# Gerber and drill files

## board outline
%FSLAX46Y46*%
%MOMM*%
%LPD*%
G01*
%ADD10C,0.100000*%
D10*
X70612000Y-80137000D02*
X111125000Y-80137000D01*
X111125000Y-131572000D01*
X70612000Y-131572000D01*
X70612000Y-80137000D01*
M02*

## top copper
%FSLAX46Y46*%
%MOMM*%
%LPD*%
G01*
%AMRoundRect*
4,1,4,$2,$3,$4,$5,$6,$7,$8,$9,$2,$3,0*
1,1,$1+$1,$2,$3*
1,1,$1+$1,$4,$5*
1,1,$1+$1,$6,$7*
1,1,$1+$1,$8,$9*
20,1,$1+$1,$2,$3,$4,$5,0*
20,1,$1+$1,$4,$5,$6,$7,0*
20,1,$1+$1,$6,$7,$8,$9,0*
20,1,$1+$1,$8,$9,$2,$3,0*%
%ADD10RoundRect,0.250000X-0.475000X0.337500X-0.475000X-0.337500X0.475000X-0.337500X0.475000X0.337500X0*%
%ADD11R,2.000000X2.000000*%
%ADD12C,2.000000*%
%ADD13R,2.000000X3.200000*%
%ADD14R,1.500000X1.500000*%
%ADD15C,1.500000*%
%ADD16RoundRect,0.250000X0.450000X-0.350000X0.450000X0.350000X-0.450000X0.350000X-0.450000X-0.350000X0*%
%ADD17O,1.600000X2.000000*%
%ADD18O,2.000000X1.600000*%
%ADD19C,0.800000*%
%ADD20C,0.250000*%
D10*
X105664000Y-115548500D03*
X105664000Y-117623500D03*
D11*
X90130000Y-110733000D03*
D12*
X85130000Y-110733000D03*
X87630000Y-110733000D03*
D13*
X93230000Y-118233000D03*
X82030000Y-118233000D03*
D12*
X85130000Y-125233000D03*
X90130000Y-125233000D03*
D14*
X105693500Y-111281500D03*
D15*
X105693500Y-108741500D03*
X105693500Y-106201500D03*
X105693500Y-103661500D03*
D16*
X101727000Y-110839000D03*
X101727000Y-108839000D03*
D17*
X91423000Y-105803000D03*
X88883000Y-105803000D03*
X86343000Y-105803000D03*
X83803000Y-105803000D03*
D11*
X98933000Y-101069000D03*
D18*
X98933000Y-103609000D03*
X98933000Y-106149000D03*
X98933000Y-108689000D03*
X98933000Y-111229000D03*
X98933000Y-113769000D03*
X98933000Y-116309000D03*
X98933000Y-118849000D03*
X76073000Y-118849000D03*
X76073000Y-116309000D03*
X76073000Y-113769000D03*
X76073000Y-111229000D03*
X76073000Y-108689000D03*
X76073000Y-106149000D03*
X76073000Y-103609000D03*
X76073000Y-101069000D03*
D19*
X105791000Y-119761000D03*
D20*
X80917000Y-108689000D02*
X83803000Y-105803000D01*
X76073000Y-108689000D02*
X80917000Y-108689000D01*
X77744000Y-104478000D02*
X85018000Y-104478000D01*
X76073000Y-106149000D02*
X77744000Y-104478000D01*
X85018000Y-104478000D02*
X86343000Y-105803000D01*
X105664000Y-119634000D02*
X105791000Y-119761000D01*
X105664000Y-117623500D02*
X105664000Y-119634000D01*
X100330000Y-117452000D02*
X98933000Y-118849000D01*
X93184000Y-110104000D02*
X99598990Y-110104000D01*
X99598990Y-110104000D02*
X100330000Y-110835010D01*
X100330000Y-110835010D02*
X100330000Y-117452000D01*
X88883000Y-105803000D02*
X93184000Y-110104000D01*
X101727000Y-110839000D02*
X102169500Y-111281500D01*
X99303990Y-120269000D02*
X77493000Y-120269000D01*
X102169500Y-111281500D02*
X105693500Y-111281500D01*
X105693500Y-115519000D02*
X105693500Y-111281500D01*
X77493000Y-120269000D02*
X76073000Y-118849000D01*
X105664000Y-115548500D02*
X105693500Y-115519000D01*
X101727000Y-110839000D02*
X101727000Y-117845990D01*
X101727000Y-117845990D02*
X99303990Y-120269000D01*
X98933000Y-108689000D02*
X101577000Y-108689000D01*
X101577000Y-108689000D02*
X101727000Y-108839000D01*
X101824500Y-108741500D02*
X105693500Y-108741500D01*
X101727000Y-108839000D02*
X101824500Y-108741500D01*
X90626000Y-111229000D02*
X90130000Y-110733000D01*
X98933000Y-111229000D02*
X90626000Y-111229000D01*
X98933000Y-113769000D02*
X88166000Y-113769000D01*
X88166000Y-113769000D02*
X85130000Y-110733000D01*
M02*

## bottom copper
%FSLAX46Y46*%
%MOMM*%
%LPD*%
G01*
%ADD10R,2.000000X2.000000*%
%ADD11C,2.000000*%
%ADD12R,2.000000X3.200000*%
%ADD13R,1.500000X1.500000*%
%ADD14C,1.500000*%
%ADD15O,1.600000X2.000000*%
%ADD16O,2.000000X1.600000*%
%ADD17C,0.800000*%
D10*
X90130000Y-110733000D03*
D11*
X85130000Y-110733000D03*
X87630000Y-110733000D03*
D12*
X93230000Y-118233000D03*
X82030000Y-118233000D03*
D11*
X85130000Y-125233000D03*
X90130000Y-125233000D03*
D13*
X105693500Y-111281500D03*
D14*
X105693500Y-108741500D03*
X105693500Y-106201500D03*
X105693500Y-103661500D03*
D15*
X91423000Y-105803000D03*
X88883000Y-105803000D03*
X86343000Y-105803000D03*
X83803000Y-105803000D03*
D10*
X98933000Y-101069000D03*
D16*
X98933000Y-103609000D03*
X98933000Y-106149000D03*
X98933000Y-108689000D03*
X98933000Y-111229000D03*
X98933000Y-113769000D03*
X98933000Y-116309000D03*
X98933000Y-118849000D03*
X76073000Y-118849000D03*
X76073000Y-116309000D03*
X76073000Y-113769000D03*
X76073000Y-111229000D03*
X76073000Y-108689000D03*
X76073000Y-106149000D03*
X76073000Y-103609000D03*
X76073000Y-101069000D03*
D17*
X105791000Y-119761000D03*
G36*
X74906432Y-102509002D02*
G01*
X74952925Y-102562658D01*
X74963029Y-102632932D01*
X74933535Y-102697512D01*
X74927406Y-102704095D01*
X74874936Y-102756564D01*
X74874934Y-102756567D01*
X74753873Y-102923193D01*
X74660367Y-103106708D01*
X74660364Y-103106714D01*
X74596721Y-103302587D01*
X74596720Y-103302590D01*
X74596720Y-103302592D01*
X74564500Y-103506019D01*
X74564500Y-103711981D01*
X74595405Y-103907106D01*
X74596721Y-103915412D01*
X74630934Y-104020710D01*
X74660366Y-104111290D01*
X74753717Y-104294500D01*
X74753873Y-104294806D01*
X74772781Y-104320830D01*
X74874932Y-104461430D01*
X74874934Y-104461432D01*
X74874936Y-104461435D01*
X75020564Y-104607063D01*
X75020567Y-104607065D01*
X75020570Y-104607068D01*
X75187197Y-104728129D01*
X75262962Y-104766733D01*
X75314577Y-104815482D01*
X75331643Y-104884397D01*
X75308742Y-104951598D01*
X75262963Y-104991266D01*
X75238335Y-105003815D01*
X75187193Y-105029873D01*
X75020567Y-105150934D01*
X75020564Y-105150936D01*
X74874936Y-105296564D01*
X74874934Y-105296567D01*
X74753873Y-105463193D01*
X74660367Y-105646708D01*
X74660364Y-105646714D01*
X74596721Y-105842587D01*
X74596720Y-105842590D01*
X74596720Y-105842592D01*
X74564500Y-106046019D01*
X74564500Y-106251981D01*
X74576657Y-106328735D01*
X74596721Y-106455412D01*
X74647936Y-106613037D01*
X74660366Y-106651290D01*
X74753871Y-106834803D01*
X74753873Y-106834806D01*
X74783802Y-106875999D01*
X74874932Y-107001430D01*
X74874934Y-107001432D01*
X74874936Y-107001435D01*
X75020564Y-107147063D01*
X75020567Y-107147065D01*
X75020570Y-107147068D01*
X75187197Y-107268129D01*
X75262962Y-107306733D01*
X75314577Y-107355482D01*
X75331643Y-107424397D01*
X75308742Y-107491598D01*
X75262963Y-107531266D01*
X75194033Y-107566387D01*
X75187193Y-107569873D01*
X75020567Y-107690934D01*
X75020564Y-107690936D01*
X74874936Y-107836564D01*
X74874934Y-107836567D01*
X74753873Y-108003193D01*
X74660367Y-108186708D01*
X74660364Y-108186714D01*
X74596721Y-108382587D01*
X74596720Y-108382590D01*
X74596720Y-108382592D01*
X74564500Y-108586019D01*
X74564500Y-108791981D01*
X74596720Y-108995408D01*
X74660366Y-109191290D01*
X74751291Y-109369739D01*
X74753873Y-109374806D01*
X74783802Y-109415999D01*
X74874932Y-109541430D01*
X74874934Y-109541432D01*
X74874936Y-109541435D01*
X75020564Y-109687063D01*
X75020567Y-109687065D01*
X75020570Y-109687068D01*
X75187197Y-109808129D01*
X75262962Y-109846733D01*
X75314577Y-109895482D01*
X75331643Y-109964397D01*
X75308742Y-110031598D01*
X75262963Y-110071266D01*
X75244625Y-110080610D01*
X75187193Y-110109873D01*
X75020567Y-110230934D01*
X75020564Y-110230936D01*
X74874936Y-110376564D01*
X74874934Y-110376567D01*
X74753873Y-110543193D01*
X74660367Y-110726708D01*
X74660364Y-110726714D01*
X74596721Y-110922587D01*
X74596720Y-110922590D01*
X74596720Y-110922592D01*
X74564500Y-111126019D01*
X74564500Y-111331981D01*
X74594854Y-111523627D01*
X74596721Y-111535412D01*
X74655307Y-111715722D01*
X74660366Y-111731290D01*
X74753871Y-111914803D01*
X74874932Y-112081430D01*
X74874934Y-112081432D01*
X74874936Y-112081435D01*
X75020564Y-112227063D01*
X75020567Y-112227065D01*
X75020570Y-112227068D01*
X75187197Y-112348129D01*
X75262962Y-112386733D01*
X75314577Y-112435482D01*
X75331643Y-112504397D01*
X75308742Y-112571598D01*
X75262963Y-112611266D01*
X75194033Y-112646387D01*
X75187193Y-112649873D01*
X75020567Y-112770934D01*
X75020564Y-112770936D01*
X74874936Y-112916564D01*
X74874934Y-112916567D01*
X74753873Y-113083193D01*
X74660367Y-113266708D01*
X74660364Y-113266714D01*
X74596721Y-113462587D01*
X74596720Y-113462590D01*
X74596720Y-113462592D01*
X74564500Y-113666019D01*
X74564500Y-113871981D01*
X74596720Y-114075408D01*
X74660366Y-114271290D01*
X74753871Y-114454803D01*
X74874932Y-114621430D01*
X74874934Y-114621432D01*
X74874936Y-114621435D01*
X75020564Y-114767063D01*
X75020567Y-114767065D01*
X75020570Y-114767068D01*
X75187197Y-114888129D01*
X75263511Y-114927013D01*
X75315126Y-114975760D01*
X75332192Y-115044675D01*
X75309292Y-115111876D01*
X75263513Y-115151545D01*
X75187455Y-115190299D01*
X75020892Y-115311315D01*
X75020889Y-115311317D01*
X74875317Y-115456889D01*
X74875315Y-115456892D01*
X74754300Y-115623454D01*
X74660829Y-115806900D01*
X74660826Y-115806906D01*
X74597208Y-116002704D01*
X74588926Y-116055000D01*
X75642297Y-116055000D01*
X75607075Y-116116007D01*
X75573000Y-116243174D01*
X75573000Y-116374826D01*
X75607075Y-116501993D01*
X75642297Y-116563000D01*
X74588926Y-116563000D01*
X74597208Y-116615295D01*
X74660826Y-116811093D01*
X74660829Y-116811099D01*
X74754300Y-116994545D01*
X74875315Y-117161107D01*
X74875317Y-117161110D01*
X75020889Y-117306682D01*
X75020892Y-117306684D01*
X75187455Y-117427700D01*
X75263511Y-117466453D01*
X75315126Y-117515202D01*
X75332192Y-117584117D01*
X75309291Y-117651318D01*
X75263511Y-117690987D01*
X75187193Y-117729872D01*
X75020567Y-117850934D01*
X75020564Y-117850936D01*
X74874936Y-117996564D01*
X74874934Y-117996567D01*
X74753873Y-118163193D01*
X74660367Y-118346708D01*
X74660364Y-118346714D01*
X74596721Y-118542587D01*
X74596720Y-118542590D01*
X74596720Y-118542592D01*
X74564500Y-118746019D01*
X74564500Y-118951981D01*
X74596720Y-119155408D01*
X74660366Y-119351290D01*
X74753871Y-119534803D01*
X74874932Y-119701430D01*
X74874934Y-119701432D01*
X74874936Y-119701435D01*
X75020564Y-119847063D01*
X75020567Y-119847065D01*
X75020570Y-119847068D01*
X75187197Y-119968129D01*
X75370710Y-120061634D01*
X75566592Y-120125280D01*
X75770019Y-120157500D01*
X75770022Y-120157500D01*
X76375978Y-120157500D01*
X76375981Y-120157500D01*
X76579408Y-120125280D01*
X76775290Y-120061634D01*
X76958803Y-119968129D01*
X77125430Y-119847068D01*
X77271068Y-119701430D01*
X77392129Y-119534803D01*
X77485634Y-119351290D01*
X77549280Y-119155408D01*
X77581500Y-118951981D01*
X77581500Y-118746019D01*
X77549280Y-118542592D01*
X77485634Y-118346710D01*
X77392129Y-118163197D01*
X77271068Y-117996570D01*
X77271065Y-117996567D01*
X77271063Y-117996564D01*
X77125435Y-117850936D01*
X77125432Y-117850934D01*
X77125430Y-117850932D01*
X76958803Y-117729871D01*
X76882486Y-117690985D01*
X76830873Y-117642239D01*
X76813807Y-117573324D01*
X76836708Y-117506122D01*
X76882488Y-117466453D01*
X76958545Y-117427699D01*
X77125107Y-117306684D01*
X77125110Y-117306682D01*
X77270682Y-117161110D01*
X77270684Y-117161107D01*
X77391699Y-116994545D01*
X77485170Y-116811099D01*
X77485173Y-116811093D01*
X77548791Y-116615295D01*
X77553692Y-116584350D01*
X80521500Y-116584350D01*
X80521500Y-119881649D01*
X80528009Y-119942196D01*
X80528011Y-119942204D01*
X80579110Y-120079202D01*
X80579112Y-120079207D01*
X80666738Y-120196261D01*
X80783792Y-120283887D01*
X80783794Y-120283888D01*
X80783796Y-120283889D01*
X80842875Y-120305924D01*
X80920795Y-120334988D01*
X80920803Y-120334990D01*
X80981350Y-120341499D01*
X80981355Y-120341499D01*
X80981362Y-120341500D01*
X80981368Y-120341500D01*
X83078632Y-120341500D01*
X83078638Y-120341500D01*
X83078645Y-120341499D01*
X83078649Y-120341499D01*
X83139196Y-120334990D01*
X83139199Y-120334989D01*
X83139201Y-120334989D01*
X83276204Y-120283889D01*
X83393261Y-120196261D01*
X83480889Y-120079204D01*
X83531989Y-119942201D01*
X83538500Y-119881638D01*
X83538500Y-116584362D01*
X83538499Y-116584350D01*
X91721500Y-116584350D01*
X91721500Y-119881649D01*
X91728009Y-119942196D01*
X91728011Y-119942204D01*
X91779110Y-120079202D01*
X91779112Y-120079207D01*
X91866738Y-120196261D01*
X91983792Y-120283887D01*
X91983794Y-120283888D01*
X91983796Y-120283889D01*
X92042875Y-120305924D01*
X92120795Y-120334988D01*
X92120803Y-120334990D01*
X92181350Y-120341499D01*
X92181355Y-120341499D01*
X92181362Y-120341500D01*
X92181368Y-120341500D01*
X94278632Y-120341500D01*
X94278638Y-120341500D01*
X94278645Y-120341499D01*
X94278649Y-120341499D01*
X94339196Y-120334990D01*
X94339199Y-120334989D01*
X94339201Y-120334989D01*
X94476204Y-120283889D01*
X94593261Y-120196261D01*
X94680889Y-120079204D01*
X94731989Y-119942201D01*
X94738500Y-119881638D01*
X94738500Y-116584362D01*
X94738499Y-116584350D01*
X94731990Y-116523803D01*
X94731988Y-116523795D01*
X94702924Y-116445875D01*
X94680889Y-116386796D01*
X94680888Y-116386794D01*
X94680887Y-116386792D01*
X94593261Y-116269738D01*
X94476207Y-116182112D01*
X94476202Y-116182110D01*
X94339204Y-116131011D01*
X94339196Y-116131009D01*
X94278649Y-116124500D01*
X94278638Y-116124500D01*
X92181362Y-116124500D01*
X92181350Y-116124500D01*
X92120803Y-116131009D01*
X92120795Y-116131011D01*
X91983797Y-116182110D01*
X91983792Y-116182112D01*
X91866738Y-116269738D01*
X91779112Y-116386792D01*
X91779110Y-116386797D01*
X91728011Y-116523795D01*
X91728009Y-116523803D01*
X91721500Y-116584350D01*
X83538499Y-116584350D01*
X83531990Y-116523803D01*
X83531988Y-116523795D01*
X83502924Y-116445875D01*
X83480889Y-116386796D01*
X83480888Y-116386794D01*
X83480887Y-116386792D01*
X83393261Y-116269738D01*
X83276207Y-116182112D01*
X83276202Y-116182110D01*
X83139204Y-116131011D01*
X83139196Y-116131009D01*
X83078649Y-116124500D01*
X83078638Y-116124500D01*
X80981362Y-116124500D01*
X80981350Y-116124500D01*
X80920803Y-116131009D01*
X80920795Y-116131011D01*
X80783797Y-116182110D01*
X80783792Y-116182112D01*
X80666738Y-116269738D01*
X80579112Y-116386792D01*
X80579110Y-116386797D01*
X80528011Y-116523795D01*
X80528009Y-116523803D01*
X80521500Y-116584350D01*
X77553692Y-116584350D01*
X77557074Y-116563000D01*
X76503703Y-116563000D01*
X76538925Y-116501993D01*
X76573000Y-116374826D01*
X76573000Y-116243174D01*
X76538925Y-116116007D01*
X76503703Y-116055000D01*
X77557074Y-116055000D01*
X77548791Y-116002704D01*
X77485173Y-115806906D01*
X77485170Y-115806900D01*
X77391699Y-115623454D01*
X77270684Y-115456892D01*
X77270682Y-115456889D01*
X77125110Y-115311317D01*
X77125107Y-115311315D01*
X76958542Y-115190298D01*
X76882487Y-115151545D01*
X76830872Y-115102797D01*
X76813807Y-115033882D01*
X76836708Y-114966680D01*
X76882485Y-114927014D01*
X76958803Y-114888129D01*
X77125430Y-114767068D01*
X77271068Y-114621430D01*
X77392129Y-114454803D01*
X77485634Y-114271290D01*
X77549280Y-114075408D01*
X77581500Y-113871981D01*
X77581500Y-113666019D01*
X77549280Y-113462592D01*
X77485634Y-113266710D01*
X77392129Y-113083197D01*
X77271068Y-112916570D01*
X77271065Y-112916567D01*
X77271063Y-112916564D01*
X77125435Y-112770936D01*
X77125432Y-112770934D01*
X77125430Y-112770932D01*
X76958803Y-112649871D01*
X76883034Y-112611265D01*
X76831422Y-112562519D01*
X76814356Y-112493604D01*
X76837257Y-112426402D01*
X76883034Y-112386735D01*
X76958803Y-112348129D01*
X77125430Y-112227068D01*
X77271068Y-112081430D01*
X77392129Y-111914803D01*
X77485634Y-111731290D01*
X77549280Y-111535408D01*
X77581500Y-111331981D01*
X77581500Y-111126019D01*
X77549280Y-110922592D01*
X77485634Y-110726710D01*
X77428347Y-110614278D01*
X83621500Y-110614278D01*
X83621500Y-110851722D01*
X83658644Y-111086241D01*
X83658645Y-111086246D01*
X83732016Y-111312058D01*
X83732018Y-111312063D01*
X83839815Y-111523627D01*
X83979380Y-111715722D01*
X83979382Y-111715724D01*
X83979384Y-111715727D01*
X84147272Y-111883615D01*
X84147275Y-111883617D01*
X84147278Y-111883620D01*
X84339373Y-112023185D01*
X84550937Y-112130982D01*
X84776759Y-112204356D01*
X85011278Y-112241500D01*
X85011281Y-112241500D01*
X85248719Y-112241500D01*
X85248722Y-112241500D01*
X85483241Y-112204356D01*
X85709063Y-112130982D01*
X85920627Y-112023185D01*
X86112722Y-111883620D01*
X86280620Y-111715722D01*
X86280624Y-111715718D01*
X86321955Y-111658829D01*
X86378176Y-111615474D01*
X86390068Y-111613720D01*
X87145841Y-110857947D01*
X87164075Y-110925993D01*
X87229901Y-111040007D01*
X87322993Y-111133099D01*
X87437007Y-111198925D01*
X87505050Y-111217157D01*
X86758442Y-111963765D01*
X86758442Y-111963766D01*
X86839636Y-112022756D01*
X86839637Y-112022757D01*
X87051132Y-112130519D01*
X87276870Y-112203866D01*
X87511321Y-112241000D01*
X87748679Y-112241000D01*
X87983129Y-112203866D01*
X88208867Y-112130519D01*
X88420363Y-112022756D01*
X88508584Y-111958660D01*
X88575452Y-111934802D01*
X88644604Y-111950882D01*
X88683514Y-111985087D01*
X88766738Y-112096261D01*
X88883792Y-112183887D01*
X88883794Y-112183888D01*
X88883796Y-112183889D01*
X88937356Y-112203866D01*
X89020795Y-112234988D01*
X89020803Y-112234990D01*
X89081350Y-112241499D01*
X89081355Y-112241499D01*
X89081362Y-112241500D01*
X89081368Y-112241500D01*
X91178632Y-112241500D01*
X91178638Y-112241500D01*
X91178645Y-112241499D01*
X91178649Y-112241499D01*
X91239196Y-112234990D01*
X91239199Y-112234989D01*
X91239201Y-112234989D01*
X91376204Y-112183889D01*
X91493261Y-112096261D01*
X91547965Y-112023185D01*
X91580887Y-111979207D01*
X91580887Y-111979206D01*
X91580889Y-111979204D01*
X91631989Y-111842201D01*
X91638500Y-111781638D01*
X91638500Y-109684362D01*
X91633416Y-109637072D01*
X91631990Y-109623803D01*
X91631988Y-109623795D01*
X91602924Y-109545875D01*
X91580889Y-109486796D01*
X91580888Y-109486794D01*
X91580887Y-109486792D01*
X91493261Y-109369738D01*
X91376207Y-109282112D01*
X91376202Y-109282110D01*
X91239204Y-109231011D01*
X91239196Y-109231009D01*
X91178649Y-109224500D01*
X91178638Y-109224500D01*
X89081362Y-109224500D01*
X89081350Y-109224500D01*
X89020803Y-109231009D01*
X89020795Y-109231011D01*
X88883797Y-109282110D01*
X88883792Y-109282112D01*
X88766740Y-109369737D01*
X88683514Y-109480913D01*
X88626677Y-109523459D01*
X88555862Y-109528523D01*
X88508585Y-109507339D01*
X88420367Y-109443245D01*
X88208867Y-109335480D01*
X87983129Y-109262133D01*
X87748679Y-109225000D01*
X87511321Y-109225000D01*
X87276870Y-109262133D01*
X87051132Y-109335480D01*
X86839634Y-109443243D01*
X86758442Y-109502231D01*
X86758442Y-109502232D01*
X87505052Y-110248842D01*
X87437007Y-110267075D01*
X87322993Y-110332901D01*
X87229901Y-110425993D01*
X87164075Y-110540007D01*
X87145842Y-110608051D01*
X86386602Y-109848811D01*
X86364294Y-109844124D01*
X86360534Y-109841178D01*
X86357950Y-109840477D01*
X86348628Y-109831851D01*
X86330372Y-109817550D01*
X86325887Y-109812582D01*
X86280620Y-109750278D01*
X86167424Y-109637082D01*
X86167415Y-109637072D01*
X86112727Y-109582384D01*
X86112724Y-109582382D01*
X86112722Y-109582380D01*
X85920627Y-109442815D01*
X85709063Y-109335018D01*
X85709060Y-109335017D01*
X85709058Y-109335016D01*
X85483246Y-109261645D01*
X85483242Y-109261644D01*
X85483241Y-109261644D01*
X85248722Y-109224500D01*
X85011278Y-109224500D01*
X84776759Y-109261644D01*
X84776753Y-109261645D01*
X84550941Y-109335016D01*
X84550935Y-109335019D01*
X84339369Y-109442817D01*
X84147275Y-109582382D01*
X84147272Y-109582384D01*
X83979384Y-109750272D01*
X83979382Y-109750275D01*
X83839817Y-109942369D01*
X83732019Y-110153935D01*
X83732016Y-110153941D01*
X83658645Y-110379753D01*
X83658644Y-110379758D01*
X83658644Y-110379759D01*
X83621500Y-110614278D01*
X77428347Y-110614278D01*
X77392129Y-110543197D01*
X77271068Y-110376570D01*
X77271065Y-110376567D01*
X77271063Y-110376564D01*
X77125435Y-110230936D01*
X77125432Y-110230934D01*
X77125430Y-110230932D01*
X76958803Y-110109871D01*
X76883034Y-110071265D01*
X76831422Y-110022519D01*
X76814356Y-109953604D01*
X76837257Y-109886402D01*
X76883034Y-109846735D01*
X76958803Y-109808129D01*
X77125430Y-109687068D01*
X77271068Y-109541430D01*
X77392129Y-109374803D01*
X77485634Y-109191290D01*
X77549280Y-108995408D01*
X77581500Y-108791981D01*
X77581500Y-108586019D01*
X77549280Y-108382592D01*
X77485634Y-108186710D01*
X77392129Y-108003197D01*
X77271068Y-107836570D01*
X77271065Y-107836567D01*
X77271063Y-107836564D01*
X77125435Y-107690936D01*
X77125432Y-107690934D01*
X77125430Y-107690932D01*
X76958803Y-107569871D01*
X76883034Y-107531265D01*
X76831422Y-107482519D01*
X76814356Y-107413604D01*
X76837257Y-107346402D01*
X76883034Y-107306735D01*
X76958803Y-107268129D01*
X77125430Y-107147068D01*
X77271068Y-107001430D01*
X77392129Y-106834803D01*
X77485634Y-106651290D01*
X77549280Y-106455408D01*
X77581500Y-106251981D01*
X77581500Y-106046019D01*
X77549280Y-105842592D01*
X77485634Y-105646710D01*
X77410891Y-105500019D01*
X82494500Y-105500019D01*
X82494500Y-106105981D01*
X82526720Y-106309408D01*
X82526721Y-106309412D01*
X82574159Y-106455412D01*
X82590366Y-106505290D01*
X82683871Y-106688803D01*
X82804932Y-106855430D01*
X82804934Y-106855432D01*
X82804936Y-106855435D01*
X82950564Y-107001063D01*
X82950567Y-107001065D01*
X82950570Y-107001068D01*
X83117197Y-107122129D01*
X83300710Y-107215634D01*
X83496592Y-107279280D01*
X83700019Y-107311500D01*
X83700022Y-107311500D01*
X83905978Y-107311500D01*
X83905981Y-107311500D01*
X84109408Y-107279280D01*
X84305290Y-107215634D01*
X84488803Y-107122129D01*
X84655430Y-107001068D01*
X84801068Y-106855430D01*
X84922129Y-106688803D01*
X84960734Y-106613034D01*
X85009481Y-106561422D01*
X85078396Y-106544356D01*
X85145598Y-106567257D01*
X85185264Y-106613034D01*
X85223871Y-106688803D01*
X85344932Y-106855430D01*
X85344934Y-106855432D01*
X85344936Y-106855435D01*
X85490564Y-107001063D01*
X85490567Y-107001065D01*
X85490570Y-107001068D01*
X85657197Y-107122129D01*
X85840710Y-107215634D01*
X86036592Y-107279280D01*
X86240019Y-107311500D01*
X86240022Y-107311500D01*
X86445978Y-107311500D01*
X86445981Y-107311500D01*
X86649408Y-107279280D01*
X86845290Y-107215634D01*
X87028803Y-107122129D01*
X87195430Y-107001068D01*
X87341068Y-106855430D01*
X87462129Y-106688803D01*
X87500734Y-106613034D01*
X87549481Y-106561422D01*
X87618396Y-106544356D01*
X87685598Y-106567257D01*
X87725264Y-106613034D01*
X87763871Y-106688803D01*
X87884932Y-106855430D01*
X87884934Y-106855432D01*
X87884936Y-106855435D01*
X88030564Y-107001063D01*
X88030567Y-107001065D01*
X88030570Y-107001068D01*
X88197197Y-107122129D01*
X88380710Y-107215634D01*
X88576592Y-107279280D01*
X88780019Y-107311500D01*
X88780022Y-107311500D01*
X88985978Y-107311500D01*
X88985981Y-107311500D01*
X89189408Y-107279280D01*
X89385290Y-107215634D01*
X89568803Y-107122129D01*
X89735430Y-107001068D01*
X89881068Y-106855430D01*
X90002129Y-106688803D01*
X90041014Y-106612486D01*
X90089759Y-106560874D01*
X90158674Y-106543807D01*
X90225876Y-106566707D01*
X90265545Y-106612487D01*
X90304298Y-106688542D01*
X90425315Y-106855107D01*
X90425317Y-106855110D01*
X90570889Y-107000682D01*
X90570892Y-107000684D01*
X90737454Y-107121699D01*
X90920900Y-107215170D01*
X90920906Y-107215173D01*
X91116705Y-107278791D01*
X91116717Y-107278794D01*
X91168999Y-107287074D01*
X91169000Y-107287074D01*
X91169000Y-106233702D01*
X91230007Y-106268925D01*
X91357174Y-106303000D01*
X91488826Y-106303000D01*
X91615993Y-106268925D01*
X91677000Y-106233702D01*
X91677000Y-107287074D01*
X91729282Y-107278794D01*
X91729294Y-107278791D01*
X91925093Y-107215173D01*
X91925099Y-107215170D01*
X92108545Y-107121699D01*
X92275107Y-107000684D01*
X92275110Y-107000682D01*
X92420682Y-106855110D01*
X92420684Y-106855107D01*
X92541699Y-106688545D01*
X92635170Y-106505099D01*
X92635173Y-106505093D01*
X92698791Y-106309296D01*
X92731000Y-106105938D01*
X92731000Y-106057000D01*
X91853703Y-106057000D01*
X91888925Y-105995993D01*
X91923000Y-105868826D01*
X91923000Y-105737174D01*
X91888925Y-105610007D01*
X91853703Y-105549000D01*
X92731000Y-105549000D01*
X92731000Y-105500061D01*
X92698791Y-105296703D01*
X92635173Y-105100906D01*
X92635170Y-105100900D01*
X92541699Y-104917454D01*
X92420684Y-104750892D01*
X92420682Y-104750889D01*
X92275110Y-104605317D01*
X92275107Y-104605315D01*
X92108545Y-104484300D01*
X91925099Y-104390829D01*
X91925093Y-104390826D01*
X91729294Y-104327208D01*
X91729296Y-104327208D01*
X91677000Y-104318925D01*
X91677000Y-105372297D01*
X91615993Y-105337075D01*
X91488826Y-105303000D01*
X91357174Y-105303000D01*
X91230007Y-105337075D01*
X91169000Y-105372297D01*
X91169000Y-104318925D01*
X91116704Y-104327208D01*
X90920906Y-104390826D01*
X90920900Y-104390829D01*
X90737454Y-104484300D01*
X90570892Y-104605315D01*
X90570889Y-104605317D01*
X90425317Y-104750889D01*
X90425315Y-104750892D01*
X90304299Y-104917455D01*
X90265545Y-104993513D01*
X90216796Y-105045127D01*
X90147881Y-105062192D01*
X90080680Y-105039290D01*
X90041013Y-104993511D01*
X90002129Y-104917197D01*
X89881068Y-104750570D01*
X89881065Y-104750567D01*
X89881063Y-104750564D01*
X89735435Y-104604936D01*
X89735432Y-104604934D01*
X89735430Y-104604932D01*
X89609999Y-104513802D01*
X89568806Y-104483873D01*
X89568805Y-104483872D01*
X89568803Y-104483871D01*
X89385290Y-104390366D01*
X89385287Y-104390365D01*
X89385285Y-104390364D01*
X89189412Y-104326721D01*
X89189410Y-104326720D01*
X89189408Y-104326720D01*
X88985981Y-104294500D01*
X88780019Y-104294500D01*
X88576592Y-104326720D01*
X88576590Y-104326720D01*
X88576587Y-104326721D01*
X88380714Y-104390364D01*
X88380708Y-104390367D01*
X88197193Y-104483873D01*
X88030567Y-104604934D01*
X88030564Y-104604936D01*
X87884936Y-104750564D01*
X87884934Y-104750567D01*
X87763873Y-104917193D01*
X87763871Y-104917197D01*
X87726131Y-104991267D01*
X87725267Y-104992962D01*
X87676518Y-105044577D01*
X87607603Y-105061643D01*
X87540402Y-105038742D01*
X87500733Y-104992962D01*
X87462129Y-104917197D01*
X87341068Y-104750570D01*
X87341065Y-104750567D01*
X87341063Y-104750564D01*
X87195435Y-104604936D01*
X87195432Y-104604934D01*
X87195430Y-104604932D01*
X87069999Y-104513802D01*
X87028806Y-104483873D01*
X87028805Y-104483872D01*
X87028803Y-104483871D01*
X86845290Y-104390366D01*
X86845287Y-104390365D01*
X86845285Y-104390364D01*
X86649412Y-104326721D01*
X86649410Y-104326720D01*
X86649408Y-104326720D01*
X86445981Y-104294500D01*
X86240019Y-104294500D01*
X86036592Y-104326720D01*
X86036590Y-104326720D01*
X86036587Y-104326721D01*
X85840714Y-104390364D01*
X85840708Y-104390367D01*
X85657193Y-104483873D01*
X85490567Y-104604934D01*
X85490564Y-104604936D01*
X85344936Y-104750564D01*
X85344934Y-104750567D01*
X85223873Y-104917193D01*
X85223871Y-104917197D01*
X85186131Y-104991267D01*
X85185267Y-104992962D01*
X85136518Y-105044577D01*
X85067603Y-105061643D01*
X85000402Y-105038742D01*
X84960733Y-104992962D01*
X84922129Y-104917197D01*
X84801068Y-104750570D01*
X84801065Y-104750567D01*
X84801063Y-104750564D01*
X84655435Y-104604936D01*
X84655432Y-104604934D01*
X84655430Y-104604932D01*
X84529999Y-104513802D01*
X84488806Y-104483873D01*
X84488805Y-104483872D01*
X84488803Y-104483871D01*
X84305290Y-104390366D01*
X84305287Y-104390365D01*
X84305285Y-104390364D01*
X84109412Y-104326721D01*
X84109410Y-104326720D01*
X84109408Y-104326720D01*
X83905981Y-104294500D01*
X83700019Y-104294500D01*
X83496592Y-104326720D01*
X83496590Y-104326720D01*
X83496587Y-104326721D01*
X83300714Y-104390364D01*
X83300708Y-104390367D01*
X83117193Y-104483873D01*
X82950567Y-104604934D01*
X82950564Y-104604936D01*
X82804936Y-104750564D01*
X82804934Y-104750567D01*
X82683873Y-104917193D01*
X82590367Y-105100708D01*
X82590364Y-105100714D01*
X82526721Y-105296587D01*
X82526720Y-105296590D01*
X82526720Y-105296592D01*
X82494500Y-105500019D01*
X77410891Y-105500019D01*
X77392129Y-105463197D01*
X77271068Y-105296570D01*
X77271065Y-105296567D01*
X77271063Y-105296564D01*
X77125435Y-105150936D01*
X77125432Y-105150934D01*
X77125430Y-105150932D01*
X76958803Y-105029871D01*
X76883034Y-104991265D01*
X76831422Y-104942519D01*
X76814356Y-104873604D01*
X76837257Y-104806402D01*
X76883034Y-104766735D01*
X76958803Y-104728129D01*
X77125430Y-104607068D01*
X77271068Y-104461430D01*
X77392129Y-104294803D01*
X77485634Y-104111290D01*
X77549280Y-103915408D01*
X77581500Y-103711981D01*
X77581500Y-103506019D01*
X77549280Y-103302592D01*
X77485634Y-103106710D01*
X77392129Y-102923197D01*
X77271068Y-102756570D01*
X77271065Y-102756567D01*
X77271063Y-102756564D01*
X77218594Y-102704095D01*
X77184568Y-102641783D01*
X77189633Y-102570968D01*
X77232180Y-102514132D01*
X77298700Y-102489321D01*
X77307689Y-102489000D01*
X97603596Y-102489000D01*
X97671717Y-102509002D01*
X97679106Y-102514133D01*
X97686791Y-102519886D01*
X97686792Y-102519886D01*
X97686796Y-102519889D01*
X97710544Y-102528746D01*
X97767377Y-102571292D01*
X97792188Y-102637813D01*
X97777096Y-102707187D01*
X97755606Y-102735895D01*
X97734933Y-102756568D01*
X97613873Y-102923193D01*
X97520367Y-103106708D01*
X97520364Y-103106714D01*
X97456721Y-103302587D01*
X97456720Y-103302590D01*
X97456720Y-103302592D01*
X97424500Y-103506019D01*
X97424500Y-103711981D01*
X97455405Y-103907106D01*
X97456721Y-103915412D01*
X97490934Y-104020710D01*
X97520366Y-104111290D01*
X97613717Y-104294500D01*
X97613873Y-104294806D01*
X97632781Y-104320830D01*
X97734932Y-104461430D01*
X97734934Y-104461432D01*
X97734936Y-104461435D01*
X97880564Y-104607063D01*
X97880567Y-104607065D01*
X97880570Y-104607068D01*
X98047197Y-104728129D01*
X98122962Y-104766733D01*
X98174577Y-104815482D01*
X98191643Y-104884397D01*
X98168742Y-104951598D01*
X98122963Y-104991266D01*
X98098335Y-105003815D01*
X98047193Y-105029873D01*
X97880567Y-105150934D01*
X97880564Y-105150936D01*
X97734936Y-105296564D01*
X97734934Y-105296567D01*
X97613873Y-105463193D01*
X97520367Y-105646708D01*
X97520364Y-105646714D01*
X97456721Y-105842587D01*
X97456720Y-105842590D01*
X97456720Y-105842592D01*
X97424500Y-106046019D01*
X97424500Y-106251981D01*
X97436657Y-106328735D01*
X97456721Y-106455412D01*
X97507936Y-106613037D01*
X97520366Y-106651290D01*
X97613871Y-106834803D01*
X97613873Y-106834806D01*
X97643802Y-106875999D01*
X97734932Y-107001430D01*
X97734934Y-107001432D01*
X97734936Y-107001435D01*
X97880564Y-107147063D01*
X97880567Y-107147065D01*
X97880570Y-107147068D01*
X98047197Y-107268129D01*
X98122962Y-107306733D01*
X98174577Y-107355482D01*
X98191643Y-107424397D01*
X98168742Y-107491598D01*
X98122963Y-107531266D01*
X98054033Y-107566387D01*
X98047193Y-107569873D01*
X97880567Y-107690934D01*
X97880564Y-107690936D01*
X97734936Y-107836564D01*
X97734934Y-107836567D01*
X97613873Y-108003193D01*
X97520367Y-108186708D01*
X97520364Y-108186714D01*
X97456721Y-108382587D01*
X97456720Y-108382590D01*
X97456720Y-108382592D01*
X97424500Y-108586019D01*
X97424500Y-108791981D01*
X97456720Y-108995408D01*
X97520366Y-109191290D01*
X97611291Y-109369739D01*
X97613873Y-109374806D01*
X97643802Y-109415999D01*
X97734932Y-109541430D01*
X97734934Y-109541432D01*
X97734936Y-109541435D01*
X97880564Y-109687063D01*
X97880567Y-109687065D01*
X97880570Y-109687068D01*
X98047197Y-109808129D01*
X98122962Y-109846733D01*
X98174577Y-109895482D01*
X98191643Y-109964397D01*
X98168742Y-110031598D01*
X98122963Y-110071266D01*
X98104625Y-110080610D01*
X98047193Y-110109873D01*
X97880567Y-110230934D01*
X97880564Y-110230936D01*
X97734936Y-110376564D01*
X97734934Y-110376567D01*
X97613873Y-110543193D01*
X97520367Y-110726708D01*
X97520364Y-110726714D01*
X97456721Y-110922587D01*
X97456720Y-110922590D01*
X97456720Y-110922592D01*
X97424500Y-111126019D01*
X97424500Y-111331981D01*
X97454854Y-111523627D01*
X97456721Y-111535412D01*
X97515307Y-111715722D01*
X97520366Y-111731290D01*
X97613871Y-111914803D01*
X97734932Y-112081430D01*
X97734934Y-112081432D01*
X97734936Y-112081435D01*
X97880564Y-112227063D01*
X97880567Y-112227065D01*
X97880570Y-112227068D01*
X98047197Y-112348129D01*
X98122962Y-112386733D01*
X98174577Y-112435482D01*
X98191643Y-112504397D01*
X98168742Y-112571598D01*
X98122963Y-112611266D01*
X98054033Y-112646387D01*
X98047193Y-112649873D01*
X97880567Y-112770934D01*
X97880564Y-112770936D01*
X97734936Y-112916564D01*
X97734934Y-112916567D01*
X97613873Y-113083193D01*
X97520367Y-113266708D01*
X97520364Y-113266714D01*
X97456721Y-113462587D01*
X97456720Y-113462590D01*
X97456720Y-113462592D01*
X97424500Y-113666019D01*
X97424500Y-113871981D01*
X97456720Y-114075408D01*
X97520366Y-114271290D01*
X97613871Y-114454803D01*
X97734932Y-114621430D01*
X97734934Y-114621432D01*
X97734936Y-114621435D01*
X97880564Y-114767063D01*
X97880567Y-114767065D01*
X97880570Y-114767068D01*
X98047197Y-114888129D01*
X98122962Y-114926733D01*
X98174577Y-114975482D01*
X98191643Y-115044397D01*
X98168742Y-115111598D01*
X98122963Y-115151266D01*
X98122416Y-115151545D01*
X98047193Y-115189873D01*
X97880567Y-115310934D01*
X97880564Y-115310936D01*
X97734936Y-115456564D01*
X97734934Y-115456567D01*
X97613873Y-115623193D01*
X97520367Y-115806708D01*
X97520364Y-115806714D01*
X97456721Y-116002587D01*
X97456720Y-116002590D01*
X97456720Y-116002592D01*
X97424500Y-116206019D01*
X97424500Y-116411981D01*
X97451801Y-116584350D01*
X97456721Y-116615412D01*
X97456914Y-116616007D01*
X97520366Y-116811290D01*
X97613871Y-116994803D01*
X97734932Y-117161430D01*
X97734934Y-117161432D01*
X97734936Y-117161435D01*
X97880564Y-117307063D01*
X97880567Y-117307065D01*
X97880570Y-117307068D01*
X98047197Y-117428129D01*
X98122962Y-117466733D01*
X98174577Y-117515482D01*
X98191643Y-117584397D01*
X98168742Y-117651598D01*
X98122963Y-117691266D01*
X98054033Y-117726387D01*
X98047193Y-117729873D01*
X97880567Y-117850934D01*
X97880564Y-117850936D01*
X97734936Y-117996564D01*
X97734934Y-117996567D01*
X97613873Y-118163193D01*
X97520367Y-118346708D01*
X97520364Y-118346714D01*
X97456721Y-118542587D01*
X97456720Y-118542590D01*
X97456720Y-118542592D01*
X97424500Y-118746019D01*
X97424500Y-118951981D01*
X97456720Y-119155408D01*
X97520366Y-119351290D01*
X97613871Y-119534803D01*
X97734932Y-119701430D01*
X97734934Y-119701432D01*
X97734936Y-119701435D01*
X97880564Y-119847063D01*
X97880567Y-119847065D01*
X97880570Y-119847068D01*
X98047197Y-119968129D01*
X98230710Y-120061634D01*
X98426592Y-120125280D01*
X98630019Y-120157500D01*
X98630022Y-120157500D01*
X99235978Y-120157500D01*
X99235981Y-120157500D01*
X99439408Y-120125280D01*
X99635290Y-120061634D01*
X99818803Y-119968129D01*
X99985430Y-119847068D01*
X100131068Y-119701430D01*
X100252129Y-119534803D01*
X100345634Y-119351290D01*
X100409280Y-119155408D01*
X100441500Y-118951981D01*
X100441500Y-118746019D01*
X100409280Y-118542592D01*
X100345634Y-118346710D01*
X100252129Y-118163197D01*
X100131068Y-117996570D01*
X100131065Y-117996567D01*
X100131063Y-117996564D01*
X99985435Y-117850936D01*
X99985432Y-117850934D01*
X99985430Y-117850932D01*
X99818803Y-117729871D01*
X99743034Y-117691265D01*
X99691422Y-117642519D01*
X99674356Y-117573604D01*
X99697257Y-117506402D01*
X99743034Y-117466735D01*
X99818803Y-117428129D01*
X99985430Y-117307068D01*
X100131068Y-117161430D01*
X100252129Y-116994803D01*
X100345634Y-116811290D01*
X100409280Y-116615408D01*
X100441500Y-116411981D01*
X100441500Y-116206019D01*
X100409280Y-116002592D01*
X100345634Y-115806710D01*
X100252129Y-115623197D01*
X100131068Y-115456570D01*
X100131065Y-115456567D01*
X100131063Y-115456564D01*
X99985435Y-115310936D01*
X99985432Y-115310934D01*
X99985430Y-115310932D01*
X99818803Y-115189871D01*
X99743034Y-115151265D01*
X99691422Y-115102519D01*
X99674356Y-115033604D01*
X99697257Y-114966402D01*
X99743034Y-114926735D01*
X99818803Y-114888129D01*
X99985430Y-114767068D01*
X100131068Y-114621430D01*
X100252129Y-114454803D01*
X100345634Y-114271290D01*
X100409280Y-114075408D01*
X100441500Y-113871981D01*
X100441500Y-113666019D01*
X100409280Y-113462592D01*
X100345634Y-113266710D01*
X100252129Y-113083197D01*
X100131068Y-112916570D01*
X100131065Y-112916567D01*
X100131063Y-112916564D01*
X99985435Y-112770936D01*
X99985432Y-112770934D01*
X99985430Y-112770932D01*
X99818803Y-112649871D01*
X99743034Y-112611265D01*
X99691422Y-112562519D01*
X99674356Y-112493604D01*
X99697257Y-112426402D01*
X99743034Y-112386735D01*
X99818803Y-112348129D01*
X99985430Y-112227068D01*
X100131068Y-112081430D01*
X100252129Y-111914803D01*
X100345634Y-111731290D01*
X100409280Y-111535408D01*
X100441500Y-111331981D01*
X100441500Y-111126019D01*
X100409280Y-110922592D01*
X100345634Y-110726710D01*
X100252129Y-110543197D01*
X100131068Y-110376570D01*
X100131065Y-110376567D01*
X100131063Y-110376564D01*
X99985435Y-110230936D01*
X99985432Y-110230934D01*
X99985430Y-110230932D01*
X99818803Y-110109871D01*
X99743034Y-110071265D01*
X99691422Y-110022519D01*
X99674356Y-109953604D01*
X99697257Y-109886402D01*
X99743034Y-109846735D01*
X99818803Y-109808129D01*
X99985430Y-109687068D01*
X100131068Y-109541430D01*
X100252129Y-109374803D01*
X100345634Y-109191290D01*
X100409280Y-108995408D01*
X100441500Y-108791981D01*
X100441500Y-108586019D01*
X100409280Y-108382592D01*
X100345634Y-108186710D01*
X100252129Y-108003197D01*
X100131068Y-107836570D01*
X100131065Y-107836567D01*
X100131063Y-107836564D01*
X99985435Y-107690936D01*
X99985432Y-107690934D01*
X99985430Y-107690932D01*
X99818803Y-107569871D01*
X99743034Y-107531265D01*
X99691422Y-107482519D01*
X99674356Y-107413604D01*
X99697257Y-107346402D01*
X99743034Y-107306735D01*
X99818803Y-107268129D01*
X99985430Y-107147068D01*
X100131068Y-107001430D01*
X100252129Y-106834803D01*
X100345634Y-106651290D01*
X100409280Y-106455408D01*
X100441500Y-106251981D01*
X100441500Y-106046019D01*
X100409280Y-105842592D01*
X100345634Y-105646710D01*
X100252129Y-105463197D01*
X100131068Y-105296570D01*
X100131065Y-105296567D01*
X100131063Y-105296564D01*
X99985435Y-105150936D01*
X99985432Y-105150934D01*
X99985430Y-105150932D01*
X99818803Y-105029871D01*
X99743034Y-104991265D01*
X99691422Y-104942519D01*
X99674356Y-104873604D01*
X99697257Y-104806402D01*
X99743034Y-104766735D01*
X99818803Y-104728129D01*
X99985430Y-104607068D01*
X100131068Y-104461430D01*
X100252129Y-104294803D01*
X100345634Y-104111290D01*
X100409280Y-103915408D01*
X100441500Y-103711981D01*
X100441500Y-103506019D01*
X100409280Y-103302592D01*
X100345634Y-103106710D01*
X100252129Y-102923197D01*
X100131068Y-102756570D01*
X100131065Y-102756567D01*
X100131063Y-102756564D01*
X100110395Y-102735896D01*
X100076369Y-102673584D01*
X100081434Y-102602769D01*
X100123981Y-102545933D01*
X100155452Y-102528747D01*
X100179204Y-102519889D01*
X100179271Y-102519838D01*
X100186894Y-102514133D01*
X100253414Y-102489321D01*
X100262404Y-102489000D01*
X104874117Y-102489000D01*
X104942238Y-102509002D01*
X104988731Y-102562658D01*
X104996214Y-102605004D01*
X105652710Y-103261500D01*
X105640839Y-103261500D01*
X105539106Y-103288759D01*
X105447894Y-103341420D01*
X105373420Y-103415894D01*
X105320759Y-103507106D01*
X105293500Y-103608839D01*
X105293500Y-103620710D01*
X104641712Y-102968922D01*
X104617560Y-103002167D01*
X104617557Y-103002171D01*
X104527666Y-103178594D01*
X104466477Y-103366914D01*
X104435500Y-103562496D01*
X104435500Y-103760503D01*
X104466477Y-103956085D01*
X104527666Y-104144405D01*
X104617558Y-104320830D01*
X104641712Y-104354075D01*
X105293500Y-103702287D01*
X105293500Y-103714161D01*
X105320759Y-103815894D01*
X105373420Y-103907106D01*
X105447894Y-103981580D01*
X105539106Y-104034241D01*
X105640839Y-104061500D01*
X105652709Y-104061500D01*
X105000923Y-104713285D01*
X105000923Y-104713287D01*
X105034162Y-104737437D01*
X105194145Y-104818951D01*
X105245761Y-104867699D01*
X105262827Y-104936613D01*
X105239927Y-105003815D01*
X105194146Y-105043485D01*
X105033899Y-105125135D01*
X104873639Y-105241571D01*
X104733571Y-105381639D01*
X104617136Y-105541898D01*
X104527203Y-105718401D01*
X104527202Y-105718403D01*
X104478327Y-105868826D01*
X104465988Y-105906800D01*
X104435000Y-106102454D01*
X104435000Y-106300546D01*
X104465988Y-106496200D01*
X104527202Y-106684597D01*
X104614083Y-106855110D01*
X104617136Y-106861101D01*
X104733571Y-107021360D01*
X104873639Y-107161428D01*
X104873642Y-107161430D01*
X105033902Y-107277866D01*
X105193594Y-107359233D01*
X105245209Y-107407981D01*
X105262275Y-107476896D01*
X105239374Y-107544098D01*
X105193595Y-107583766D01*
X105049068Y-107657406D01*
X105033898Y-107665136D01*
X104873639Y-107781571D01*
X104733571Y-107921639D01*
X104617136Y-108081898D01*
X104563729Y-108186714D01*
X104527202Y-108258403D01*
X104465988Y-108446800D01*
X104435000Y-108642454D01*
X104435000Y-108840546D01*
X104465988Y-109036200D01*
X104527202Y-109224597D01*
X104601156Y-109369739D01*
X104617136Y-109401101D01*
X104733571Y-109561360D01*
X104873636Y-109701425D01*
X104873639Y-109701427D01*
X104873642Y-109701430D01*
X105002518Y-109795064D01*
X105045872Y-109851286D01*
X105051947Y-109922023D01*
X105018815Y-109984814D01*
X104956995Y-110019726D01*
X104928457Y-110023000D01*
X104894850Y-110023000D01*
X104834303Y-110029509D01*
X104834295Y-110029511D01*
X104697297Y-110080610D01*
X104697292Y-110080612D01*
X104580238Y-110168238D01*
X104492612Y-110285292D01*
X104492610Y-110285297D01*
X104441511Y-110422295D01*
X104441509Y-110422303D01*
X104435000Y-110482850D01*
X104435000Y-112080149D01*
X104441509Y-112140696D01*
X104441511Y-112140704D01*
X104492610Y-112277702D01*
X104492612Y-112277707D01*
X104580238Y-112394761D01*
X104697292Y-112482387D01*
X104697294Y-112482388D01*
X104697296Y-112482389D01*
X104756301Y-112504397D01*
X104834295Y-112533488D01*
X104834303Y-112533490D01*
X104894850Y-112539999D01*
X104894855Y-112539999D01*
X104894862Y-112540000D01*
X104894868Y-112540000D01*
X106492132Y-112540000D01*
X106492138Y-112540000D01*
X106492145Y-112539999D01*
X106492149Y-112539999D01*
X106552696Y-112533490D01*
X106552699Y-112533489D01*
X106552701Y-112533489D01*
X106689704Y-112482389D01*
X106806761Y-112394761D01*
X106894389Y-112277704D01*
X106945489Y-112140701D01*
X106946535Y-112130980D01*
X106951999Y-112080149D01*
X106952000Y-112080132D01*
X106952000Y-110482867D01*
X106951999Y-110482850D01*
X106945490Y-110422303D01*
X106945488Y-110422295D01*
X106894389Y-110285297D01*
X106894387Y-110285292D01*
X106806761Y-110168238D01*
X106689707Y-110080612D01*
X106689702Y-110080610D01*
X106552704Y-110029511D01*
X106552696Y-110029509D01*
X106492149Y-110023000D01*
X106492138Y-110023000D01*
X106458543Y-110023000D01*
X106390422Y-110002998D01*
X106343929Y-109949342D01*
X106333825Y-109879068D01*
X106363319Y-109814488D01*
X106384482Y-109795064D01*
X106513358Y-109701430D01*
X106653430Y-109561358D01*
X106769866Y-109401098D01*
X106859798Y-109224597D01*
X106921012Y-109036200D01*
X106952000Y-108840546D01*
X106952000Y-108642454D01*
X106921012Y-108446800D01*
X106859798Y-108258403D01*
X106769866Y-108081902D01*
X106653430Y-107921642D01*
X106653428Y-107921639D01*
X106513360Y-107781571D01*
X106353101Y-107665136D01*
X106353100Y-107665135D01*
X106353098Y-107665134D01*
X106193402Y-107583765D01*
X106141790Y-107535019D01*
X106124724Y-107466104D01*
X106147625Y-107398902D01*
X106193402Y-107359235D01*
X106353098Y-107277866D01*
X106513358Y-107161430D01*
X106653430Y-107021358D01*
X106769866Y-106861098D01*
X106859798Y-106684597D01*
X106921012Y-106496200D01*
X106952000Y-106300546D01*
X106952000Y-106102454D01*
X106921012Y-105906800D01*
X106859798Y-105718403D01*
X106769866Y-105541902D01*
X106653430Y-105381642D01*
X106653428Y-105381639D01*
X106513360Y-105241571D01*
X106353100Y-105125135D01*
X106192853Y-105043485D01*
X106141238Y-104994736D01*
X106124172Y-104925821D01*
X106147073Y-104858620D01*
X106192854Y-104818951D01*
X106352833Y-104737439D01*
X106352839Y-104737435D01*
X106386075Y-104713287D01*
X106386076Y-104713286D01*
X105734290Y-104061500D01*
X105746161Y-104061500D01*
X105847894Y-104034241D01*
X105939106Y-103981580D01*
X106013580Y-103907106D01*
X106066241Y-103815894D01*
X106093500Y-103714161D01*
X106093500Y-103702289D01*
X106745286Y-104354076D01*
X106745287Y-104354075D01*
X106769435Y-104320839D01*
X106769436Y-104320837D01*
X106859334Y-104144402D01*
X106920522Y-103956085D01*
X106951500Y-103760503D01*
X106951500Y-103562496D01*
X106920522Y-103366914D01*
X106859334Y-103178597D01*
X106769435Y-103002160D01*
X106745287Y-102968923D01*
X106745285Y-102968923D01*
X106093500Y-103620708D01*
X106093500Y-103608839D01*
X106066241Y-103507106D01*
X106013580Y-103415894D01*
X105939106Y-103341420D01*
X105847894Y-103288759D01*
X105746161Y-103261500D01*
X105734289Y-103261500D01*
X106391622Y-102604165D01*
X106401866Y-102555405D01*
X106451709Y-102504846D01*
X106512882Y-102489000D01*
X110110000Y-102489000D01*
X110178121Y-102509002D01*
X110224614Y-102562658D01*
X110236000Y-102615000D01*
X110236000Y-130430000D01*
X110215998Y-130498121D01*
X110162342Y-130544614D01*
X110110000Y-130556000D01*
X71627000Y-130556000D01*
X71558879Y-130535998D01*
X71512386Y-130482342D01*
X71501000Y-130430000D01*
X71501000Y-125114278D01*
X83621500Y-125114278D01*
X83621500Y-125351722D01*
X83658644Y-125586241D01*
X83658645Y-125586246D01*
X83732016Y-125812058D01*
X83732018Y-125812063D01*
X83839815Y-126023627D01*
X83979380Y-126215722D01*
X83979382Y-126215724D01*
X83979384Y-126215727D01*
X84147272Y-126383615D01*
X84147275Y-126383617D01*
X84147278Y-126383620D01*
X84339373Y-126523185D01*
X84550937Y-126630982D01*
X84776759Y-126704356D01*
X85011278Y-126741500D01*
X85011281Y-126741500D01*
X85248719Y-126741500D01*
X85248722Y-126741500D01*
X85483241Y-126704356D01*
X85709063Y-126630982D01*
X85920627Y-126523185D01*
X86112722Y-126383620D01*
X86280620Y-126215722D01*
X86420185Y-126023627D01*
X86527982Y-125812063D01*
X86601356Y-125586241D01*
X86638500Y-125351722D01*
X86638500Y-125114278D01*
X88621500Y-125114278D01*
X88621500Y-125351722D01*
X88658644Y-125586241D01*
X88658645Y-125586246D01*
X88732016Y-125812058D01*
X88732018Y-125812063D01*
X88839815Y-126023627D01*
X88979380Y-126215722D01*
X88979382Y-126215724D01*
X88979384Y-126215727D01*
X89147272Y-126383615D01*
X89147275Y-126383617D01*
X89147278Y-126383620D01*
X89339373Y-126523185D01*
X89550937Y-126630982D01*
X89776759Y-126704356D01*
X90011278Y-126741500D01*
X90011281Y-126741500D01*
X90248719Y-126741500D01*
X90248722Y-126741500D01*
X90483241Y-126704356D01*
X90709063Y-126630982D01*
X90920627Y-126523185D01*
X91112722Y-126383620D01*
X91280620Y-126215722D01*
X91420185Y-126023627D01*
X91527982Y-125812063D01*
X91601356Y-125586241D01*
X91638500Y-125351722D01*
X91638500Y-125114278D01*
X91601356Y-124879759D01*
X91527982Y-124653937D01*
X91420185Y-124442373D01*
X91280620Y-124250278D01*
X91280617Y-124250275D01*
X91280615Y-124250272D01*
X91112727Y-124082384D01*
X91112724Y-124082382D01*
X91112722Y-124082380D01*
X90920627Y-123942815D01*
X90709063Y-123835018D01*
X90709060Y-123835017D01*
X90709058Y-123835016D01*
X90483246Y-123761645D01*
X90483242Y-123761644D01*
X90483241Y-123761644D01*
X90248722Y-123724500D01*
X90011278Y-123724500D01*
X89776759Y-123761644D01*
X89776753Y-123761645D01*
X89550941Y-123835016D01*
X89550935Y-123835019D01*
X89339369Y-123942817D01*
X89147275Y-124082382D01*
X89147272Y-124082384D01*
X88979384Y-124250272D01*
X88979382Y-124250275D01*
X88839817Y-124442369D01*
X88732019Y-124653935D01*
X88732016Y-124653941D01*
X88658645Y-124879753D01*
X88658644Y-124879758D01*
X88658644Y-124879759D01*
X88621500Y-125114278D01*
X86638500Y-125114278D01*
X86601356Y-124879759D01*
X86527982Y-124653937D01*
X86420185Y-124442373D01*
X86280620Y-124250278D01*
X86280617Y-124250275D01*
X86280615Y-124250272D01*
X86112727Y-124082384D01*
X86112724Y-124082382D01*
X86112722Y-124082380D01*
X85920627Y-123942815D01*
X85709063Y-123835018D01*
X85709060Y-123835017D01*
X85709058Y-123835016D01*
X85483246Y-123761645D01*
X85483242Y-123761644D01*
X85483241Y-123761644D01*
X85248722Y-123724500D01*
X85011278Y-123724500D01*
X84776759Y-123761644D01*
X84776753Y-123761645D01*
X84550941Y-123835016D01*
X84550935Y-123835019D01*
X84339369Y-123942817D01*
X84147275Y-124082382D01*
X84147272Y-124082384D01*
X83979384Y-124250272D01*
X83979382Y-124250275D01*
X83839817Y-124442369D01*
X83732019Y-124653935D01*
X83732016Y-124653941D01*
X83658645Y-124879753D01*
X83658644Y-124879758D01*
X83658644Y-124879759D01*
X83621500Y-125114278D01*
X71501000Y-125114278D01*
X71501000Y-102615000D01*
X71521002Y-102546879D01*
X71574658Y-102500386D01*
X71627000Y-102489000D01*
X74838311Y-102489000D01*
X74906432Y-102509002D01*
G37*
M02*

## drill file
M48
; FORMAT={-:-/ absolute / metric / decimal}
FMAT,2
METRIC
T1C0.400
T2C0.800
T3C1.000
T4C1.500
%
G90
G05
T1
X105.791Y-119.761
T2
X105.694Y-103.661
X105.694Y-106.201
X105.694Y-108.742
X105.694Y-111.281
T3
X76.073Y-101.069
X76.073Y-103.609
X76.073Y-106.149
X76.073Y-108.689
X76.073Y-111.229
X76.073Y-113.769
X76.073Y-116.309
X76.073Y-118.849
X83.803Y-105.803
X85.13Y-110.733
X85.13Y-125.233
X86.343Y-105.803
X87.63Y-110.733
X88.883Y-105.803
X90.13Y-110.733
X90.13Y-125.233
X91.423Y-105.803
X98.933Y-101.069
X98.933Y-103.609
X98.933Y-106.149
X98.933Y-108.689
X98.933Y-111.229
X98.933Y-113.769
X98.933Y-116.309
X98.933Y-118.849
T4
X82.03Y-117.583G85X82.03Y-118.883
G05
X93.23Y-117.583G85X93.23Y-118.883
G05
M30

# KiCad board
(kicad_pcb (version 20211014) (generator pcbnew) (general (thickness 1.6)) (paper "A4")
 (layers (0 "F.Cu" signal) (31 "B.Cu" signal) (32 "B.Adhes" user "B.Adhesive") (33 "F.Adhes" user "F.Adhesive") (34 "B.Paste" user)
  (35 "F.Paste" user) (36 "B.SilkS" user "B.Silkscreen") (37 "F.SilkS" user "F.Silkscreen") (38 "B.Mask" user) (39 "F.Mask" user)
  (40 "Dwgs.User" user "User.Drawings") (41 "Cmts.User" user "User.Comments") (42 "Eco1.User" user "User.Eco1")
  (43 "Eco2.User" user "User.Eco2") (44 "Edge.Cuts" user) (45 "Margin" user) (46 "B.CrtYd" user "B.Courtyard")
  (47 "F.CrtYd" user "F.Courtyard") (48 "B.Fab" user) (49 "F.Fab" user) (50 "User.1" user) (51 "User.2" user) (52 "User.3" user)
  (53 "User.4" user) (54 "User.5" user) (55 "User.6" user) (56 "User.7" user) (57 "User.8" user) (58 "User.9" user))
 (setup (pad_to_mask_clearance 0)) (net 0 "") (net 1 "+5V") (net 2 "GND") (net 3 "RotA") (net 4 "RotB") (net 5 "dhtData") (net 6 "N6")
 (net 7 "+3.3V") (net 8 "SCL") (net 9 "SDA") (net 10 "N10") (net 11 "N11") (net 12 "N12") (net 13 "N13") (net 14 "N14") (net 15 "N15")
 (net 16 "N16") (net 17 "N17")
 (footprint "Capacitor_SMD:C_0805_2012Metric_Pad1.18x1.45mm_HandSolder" (layer "F.Cu") (at 105.664 116.586 -90)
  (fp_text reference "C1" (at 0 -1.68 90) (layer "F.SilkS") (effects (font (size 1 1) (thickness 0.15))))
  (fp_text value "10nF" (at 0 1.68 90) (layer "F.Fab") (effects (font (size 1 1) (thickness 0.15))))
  (pad "1" smd roundrect (at -1.0375 0 270) (size 1.175 1.45) (layers "F.Cu" "F.Paste" "F.Mask") (roundrect_rratio 0.212766) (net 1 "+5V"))
  (pad "2" smd roundrect (at 1.0375 0 270) (size 1.175 1.45) (layers "F.Cu" "F.Paste" "F.Mask") (roundrect_rratio 0.212766) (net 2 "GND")))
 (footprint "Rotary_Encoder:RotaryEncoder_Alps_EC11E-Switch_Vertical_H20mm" (layer "F.Cu") (at 90.13 110.733 -90)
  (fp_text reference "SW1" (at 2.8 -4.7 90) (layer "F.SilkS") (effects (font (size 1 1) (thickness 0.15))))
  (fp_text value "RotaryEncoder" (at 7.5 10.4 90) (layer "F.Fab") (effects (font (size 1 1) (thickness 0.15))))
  (pad "A" thru_hole rect (at 0 0 270) (size 2 2) (drill 1) (layers *.Cu *.Mask) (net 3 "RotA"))
  (pad "B" thru_hole circle (at 0 5 270) (size 2 2) (drill 1) (layers *.Cu *.Mask) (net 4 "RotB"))
  (pad "C" thru_hole circle (at 0 2.5 270) (size 2 2) (drill 1) (layers *.Cu *.Mask) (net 2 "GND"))
  (pad "MP" thru_hole rect (at 7.5 -3.1 270) (size 3.2 2) (drill oval 2.8 1.5) (layers *.Cu *.Mask))
  (pad "MP" thru_hole rect (at 7.5 8.1 270) (size 3.2 2) (drill oval 2.8 1.5) (layers *.Cu *.Mask))
  (pad "S1" thru_hole circle (at 14.5 5 270) (size 2 2) (drill 1) (layers *.Cu *.Mask))
  (pad "S2" thru_hole circle (at 14.5 0 270) (size 2 2) (drill 1) (layers *.Cu *.Mask)))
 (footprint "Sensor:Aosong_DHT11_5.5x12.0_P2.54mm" (layer "F.Cu") (at 105.6935 111.2815 180)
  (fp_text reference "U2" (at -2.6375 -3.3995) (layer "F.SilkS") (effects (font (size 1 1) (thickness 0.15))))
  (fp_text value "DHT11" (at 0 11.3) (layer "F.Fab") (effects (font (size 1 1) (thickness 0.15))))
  (pad "1" thru_hole rect (at 0 0 180) (size 1.5 1.5) (drill 0.8) (layers *.Cu *.Mask) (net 1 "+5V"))
  (pad "2" thru_hole circle (at 0 2.54 180) (size 1.5 1.5) (drill 0.8) (layers *.Cu *.Mask) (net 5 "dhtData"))
  (pad "3" thru_hole circle (at 0 5.08 180) (size 1.5 1.5) (drill 0.8) (layers *.Cu *.Mask) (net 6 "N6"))
  (pad "4" thru_hole circle (at 0 7.62 180) (size 1.5 1.5) (drill 0.8) (layers *.Cu *.Mask) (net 2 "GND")))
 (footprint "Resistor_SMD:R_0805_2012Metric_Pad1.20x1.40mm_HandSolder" (layer "F.Cu") (at 101.727 109.839 90)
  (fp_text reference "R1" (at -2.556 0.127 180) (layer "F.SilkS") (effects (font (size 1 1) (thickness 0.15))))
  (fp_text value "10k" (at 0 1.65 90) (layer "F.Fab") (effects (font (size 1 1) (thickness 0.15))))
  (pad "1" smd roundrect (at -1 0 90) (size 1.2 1.4) (layers "F.Cu" "F.Paste" "F.Mask") (roundrect_rratio 0.208333) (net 1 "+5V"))
  (pad "2" smd roundrect (at 1 0 90) (size 1.2 1.4) (layers "F.Cu" "F.Paste" "F.Mask") (roundrect_rratio 0.208333) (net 5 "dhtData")))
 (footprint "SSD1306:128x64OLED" (layer "F.Cu") (at 87.803 95.203 180)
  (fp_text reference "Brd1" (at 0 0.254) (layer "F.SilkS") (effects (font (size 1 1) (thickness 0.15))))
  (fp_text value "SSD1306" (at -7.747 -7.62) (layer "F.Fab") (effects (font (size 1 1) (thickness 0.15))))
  (pad "1" thru_hole oval locked (at -3.62 -10.6 270) (size 2 1.6) (drill 1) (layers *.Cu *.Mask) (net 2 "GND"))
  (pad "2" thru_hole oval locked (at -1.08 -10.6 270) (size 2 1.6) (drill 1) (layers *.Cu *.Mask) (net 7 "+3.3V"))
  (pad "3" thru_hole oval locked (at 1.46 -10.6 270) (size 2 1.6) (drill 1) (layers *.Cu *.Mask) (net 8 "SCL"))
  (pad "4" thru_hole oval locked (at 4 -10.6 270) (size 2 1.6) (drill 1) (layers *.Cu *.Mask) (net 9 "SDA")))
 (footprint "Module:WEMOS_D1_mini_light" (layer "B.Cu") (at 98.933 101.069 180)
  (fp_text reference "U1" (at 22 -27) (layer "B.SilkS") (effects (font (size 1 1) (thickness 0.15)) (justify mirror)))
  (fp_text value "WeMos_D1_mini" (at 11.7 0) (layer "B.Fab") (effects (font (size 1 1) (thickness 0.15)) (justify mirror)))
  (pad "1" thru_hole rect (at 0 0 180) (size 2 2) (drill 1) (layers *.Cu *.Mask) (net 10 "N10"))
  (pad "2" thru_hole oval (at 0 -2.54 180) (size 2 1.6) (drill 1) (layers *.Cu *.Mask) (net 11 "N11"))
  (pad "3" thru_hole oval (at 0 -5.08 180) (size 2 1.6) (drill 1) (layers *.Cu *.Mask) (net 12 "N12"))
  (pad "4" thru_hole oval (at 0 -7.62 180) (size 2 1.6) (drill 1) (layers *.Cu *.Mask) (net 5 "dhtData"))
  (pad "5" thru_hole oval (at 0 -10.16 180) (size 2 1.6) (drill 1) (layers *.Cu *.Mask) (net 3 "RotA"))
  (pad "6" thru_hole oval (at 0 -12.7 180) (size 2 1.6) (drill 1) (layers *.Cu *.Mask) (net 4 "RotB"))
  (pad "7" thru_hole oval (at 0 -15.24 180) (size 2 1.6) (drill 1) (layers *.Cu *.Mask) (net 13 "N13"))
  (pad "8" thru_hole oval (at 0 -17.78 180) (size 2 1.6) (drill 1) (layers *.Cu *.Mask) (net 7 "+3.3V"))
  (pad "9" thru_hole oval (at 22.86 -17.78 180) (size 2 1.6) (drill 1) (layers *.Cu *.Mask) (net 1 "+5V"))
  (pad "10" thru_hole oval (at 22.86 -15.24 180) (size 2 1.6) (drill 1) (layers *.Cu *.Mask) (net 2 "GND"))
  (pad "11" thru_hole oval (at 22.86 -12.7 180) (size 2 1.6) (drill 1) (layers *.Cu *.Mask) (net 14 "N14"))
  (pad "12" thru_hole oval (at 22.86 -10.16 180) (size 2 1.6) (drill 1) (layers *.Cu *.Mask) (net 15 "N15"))
  (pad "13" thru_hole oval (at 22.86 -7.62 180) (size 2 1.6) (drill 1) (layers *.Cu *.Mask) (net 9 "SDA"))
  (pad "14" thru_hole oval (at 22.86 -5.08 180) (size 2 1.6) (drill 1) (layers *.Cu *.Mask) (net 8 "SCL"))
  (pad "15" thru_hole oval (at 22.86 -2.54 180) (size 2 1.6) (drill 1) (layers *.Cu *.Mask) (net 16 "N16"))
  (pad "16" thru_hole oval (at 22.86 0 180) (size 2 1.6) (drill 1) (layers *.Cu *.Mask) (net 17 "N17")))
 (gr_rect (start 70.612 80.137) (end 111.125 131.572) (layer "Edge.Cuts") (width 0.1) (fill none))
 (segment (start 80.917 108.689) (end 83.803 105.803) (width 0.25) (layer "F.Cu") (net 9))
 (segment (start 76.073 108.689) (end 80.917 108.689) (width 0.25) (layer "F.Cu") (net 9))
 (segment (start 77.744 104.478) (end 85.018 104.478) (width 0.25) (layer "F.Cu") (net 8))
 (segment (start 76.073 106.149) (end 77.744 104.478) (width 0.25) (layer "F.Cu") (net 8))
 (segment (start 85.018 104.478) (end 86.343 105.803) (width 0.25) (layer "F.Cu") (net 8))
 (segment (start 105.664 119.634) (end 105.791 119.761) (width 0.25) (layer "F.Cu") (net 2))
 (segment (start 105.664 117.6235) (end 105.664 119.634) (width 0.25) (layer "F.Cu") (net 2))
 (via (at 105.791 119.761) (size 0.8) (drill 0.4) (layers "F.Cu" "B.Cu") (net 2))
 (segment (start 100.33 117.452) (end 98.933 118.849) (width 0.25) (layer "F.Cu") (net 7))
 (segment (start 93.184 110.104) (end 99.59899 110.104) (width 0.25) (layer "F.Cu") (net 7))
 (segment (start 99.59899 110.104) (end 100.33 110.83501) (width 0.25) (layer "F.Cu") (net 7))
 (segment (start 100.33 110.83501) (end 100.33 117.452) (width 0.25) (layer "F.Cu") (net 7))
 (segment (start 88.883 105.803) (end 93.184 110.104) (width 0.25) (layer "F.Cu") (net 7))
 (segment (start 101.727 110.839) (end 102.1695 111.2815) (width 0.25) (layer "F.Cu") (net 1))
 (segment (start 99.30399 120.269) (end 77.493 120.269) (width 0.25) (layer "F.Cu") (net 1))
 (segment (start 102.1695 111.2815) (end 105.6935 111.2815) (width 0.25) (layer "F.Cu") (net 1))
 (segment (start 105.6935 115.519) (end 105.6935 111.2815) (width 0.25) (layer "F.Cu") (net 1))
 (segment (start 77.493 120.269) (end 76.073 118.849) (width 0.25) (layer "F.Cu") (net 1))
 (segment (start 105.664 115.5485) (end 105.6935 115.519) (width 0.25) (layer "F.Cu") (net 1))
 (segment (start 101.727 110.839) (end 101.727 117.84599) (width 0.25) (layer "F.Cu") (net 1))
 (segment (start 101.727 117.84599) (end 99.30399 120.269) (width 0.25) (layer "F.Cu") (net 1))
 (segment (start 98.933 108.689) (end 101.577 108.689) (width 0.25) (layer "F.Cu") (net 5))
 (segment (start 101.577 108.689) (end 101.727 108.839) (width 0.25) (layer "F.Cu") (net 5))
 (segment (start 101.8245 108.7415) (end 105.6935 108.7415) (width 0.25) (layer "F.Cu") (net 5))
 (segment (start 101.727 108.839) (end 101.8245 108.7415) (width 0.25) (layer "F.Cu") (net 5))
 (segment (start 90.626 111.229) (end 90.13 110.733) (width 0.25) (layer "F.Cu") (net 3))
 (segment (start 98.933 111.229) (end 90.626 111.229) (width 0.25) (layer "F.Cu") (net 3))
 (segment (start 98.933 113.769) (end 88.166 113.769) (width 0.25) (layer "F.Cu") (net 4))
 (segment (start 88.166 113.769) (end 85.13 110.733) (width 0.25) (layer "F.Cu") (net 4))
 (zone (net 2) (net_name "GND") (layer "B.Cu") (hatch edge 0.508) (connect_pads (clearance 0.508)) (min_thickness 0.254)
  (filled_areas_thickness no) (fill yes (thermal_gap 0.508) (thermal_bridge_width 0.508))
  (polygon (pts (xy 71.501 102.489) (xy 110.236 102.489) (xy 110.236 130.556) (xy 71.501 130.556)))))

